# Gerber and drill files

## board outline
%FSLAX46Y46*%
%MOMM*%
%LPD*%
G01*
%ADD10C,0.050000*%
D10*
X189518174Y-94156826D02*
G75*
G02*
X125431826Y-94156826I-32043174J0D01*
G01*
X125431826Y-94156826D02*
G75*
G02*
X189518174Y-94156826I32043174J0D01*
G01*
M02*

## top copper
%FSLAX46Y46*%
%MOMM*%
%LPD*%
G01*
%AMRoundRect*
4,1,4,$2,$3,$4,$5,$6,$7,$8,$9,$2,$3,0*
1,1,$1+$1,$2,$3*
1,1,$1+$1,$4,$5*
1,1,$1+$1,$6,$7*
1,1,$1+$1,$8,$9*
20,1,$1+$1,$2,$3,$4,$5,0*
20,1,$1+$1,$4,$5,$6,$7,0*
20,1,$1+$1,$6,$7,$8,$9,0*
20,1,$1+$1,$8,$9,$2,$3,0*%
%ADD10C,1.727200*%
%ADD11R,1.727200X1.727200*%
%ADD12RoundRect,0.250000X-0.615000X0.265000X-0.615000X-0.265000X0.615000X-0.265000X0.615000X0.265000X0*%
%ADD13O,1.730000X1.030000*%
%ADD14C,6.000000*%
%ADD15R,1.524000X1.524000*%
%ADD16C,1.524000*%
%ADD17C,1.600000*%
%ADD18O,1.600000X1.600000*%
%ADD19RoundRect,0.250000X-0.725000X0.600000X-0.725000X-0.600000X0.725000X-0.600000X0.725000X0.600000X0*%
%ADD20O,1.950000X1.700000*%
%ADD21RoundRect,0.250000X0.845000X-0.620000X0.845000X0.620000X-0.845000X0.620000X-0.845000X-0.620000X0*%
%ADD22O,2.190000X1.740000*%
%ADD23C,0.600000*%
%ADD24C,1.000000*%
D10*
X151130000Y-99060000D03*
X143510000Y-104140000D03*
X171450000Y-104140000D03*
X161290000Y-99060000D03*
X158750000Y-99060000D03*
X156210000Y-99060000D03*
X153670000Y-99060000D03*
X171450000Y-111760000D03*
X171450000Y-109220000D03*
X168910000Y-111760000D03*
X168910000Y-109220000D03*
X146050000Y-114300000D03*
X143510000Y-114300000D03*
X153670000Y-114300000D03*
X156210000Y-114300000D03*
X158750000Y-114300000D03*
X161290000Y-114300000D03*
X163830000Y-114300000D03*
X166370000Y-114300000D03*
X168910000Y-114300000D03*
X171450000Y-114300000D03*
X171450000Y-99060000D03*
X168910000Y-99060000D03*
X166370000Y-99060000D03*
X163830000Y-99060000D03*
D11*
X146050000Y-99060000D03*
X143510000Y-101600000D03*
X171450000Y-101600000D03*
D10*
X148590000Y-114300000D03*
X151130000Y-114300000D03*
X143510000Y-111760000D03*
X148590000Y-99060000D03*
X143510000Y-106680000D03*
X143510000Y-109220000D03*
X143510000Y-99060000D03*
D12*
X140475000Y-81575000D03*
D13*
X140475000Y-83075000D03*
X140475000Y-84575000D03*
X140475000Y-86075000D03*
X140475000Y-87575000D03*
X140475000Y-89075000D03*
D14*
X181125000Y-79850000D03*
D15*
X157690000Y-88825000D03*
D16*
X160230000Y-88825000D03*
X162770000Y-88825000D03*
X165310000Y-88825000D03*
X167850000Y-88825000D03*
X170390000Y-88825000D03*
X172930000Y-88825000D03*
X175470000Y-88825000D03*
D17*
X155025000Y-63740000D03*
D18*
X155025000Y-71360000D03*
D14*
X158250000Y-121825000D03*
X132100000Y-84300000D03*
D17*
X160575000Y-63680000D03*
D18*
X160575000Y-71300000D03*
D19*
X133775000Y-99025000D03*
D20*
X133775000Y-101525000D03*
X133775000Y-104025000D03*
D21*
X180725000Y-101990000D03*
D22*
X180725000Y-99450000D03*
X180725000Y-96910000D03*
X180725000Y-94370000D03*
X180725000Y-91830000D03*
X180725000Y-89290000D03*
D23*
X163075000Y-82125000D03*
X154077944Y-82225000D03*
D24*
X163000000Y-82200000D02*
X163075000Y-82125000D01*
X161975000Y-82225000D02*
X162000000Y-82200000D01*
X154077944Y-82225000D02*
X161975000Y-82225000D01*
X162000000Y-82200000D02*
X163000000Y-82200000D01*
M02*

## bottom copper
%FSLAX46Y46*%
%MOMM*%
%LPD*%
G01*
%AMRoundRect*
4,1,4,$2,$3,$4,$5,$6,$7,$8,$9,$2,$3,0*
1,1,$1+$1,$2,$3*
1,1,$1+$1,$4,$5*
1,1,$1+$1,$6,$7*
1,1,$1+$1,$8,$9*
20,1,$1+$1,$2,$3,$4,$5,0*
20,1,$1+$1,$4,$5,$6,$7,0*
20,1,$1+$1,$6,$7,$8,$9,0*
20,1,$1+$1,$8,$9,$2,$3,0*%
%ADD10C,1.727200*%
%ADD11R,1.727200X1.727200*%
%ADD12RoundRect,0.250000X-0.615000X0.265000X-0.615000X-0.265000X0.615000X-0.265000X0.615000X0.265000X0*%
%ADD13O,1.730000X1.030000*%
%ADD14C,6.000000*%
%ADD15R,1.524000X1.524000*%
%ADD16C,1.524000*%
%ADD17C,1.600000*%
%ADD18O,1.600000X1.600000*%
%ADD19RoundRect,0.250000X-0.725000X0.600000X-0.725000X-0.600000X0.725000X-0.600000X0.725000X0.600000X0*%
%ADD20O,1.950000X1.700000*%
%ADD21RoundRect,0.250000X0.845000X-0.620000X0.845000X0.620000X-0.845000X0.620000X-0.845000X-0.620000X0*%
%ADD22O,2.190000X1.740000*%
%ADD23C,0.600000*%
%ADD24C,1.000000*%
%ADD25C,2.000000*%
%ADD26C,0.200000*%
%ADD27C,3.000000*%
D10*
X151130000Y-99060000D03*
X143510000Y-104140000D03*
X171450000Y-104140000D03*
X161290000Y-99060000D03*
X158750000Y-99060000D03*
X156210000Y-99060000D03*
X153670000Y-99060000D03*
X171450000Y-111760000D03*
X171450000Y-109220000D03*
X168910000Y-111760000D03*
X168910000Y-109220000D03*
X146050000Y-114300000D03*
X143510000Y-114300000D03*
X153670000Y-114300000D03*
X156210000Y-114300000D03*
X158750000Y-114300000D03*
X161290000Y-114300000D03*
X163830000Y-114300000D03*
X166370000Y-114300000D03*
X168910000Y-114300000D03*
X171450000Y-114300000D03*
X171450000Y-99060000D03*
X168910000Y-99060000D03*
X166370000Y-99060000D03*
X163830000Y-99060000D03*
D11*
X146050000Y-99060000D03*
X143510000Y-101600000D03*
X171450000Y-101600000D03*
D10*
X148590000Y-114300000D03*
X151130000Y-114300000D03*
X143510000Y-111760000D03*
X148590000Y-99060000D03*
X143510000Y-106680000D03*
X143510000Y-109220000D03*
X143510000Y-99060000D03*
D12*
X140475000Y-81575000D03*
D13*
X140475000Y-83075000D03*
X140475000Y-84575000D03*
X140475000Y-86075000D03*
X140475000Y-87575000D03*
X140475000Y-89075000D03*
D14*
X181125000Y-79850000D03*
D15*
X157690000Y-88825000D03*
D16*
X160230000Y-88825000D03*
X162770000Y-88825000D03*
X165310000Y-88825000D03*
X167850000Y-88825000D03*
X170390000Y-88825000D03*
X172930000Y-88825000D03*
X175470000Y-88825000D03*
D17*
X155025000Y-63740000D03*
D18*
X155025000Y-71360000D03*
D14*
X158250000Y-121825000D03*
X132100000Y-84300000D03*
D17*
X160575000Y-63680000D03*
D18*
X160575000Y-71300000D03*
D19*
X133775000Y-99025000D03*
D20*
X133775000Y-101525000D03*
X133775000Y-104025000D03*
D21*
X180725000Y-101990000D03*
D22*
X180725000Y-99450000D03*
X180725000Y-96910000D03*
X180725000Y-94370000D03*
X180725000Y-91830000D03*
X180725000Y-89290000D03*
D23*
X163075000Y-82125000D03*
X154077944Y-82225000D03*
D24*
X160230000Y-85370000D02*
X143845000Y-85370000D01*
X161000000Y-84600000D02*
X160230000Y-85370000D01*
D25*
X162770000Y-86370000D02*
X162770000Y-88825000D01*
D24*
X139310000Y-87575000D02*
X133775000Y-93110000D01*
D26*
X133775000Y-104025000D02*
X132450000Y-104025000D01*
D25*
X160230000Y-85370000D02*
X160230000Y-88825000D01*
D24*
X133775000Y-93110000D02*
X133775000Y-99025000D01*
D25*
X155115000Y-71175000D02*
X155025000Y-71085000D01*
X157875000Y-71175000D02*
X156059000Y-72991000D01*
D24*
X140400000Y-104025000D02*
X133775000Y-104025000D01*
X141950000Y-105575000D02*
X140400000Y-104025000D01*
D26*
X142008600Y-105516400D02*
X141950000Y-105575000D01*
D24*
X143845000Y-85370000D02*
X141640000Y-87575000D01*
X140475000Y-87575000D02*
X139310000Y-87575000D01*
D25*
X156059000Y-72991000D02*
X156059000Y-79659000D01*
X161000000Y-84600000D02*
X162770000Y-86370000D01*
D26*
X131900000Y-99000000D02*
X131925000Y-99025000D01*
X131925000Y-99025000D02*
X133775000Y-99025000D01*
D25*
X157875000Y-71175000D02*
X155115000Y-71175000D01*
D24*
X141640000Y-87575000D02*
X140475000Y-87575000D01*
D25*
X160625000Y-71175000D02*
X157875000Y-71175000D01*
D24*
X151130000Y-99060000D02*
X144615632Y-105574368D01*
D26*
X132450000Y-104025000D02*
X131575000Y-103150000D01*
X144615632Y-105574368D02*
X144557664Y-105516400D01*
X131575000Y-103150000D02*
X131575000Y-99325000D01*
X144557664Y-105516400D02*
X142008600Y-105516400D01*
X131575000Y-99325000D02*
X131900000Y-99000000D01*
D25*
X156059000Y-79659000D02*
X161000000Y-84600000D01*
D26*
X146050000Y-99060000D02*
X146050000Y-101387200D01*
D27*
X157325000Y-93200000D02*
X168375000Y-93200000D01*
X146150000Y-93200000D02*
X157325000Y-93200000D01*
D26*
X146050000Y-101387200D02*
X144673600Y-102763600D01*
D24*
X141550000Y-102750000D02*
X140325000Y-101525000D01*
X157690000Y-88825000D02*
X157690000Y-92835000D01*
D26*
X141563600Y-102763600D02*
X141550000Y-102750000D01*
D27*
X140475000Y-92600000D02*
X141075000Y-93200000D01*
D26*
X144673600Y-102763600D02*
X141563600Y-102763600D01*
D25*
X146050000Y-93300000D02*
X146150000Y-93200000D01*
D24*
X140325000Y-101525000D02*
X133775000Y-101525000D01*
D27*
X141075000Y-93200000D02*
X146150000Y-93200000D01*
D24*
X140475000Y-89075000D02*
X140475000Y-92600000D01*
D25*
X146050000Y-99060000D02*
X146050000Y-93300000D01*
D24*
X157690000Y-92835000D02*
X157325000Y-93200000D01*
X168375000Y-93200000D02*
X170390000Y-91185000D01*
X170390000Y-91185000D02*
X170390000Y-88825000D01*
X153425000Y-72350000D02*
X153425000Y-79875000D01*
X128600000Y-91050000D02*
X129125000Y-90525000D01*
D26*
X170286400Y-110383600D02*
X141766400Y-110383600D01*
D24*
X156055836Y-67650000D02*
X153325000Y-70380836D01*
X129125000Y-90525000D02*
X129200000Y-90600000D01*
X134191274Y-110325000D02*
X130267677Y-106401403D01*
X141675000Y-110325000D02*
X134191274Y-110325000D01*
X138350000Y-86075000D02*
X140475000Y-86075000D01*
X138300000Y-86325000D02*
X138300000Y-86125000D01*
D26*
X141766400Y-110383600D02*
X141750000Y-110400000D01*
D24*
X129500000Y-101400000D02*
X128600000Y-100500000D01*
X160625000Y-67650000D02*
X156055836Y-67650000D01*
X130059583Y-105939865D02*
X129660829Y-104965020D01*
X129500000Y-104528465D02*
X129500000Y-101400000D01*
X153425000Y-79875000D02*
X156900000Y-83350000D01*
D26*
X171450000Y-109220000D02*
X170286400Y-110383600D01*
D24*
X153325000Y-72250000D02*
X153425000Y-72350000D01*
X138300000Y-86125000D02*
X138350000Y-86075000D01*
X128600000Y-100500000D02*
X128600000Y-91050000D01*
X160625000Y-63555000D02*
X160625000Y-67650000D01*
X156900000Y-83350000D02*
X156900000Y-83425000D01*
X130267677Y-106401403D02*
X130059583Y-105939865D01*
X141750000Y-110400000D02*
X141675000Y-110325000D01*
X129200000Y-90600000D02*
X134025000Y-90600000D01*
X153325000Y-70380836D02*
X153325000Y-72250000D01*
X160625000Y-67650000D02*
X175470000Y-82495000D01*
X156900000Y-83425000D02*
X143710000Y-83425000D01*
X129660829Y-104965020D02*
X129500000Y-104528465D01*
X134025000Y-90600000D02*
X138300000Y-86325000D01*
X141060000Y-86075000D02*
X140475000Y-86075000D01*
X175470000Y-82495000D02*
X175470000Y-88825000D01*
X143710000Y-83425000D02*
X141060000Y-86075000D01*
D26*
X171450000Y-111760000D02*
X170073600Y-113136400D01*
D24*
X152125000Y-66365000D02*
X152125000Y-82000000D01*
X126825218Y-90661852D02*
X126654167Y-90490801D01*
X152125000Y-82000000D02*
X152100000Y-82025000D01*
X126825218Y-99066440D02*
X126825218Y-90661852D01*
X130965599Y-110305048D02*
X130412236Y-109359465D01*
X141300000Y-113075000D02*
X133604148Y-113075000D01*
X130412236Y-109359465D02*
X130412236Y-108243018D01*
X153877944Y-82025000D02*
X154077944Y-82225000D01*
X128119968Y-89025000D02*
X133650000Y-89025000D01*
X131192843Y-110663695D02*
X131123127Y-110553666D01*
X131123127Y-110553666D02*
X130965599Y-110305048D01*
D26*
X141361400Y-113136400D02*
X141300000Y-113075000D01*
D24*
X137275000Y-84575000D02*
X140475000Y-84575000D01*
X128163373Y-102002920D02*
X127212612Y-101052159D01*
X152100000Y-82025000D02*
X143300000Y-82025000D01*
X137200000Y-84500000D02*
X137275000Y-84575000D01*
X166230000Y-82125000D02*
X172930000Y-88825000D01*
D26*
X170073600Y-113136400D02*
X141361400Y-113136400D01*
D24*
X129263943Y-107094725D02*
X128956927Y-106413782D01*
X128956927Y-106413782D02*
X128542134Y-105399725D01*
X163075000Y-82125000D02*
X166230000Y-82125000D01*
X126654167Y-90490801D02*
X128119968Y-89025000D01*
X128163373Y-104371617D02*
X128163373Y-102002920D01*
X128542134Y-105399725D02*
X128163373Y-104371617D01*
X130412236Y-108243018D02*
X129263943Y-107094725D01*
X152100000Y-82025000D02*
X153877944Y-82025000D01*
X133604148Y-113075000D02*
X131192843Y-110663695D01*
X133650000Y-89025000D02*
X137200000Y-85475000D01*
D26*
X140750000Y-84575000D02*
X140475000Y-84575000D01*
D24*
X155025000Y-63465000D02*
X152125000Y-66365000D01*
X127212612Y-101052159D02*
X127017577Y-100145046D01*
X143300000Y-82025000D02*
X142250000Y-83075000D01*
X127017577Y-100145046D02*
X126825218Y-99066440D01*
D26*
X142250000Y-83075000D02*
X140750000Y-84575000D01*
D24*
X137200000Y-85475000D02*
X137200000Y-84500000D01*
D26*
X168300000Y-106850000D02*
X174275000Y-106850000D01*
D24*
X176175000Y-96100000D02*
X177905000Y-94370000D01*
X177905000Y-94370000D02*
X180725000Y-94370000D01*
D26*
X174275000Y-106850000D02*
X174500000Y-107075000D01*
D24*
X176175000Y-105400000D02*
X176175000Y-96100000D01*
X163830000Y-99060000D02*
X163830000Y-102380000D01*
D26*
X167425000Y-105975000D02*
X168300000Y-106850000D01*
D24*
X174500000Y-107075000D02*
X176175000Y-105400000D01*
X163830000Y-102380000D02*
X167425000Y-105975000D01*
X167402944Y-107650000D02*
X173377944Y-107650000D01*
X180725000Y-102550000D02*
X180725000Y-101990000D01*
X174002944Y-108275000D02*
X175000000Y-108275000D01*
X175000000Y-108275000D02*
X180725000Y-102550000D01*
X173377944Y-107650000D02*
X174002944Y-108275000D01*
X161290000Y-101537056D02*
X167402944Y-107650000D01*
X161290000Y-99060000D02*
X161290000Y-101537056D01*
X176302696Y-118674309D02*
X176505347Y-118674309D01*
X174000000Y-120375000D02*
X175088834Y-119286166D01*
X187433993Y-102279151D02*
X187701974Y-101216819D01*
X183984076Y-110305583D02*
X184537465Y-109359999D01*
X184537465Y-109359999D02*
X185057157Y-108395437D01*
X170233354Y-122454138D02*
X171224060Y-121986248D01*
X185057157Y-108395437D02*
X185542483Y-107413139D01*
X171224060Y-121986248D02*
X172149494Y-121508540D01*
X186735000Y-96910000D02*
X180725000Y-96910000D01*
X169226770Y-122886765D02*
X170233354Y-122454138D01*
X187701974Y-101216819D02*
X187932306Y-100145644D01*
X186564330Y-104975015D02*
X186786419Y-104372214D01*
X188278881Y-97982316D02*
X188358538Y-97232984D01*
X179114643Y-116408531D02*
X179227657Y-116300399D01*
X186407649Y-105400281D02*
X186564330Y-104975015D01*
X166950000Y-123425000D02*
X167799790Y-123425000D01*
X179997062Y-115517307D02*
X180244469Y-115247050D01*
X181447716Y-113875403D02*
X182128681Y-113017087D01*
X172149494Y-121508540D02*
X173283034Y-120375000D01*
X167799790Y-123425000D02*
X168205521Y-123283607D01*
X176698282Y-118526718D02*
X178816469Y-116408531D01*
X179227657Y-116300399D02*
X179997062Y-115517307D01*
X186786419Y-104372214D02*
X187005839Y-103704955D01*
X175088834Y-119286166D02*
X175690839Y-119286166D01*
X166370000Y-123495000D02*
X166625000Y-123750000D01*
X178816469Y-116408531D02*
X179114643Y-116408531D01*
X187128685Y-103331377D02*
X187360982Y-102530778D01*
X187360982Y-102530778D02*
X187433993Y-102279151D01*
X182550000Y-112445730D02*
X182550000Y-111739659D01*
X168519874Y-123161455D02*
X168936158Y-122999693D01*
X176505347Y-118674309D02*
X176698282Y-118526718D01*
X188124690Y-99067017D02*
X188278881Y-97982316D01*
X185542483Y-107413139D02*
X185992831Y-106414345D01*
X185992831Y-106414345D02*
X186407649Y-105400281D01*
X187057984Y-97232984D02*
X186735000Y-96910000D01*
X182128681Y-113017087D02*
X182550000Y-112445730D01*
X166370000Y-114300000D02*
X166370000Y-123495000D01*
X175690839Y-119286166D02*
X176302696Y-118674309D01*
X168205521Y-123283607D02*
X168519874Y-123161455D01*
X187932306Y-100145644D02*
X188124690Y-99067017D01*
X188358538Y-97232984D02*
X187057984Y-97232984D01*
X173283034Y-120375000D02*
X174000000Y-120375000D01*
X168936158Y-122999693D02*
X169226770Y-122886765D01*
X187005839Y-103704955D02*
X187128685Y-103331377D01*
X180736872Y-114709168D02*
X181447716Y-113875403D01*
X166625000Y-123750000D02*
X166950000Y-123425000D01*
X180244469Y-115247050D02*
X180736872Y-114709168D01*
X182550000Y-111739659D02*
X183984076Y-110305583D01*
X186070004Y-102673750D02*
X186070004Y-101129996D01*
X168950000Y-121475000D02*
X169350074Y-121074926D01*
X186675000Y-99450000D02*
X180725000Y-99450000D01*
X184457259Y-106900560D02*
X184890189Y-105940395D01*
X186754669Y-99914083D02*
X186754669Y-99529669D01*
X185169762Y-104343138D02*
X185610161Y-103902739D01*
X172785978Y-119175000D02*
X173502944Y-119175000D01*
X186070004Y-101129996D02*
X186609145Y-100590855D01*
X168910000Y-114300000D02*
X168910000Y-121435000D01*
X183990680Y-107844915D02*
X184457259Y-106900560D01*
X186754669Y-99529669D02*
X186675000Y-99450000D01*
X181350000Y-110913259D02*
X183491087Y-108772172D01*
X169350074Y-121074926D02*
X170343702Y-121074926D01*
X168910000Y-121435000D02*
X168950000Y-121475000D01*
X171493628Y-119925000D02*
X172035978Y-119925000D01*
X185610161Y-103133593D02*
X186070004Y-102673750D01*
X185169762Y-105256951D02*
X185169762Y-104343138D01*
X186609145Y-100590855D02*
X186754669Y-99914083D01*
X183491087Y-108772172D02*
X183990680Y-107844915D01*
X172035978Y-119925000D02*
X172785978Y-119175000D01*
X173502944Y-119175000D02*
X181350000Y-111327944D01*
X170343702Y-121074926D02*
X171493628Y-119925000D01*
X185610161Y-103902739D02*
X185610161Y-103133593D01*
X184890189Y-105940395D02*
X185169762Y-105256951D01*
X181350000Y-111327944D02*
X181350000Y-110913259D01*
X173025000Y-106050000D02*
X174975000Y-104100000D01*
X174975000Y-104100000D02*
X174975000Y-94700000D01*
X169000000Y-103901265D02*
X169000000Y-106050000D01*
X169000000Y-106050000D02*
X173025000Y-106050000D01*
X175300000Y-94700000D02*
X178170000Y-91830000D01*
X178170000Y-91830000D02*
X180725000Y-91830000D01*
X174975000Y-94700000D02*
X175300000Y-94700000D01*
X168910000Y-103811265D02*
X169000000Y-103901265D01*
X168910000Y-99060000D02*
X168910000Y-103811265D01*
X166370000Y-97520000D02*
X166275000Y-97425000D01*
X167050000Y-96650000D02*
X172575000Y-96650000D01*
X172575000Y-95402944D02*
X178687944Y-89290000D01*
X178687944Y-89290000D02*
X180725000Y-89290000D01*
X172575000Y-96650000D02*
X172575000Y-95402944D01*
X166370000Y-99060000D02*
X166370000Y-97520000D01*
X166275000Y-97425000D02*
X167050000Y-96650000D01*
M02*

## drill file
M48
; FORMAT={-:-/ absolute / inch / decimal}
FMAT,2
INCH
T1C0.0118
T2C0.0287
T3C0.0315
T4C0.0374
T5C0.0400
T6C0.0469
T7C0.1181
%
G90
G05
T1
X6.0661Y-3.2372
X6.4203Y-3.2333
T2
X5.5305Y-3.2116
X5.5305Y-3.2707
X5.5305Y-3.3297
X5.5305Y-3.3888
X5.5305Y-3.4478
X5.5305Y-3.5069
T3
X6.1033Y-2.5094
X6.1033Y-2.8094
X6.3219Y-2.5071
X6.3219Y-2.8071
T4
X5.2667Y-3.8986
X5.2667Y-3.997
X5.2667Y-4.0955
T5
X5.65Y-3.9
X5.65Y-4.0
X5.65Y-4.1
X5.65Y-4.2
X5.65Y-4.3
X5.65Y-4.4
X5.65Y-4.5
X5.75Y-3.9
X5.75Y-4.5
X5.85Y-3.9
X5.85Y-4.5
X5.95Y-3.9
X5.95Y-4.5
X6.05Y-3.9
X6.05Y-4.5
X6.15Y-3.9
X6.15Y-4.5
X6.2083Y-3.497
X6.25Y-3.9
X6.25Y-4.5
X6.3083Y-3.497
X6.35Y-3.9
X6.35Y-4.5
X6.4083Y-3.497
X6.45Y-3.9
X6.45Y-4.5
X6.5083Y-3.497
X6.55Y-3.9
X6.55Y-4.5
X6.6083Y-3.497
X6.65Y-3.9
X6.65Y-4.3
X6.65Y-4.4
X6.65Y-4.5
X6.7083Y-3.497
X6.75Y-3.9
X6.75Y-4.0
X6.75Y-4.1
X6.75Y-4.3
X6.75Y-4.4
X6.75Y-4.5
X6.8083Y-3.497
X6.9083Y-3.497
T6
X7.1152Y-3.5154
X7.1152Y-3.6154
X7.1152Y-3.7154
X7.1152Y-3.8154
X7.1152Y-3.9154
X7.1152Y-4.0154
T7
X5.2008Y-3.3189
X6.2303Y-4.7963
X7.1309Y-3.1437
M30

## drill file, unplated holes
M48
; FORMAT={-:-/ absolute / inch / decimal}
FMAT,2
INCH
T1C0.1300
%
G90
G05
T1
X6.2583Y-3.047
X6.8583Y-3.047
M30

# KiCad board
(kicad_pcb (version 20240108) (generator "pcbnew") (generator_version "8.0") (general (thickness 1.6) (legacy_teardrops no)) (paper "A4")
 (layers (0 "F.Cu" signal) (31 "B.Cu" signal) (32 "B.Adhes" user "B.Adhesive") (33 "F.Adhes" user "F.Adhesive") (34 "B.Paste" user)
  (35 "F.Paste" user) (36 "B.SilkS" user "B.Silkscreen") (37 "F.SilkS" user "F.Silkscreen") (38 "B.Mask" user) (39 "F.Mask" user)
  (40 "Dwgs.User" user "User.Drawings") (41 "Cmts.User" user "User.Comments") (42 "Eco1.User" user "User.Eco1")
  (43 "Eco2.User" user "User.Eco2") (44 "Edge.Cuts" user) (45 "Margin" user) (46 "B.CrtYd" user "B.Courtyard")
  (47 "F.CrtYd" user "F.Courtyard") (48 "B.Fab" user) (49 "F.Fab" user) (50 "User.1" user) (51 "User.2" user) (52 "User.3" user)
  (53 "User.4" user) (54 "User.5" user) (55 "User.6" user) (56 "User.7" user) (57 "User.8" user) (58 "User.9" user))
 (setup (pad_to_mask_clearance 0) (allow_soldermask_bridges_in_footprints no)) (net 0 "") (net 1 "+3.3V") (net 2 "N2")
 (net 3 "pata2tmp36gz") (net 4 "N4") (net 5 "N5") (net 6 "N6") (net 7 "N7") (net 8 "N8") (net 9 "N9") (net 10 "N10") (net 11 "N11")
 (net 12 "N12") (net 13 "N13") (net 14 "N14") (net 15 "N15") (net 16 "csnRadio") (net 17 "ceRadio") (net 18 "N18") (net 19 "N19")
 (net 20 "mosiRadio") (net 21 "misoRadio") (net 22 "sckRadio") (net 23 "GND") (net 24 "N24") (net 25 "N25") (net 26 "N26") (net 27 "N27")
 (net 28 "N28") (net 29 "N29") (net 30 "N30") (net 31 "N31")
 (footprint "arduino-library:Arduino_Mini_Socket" (layer "F.Cu") (at 172.72 115.57 90)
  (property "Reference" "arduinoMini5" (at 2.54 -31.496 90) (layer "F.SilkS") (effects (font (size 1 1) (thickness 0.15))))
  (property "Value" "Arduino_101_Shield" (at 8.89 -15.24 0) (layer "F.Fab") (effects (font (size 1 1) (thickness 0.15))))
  (pad "5V1" thru_hole circle (at 16.51 -21.59 90) (size 1.7272 1.7272) (drill 1.016) (layers "*.Cu" "*.Mask") (remove_unused_layers no)
   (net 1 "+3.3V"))
  (pad "5V2" thru_hole circle (at 11.43 -29.21 90) (size 1.7272 1.7272) (drill 1.016) (layers "*.Cu" "*.Mask") (remove_unused_layers no)
   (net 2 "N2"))
  (pad "5V3" thru_hole circle (at 11.43 -1.27 90) (size 1.7272 1.7272) (drill 1.016) (layers "*.Cu" "*.Mask") (remove_unused_layers no))
  (pad "A0" thru_hole circle (at 16.51 -11.43 90) (size 1.7272 1.7272) (drill 1.016) (layers "*.Cu" "*.Mask") (remove_unused_layers no)
   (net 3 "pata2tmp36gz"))
  (pad "A1" thru_hole circle (at 16.51 -13.97 90) (size 1.7272 1.7272) (drill 1.016) (layers "*.Cu" "*.Mask") (remove_unused_layers no)
   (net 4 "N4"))
  (pad "A2" thru_hole circle (at 16.51 -16.51 90) (size 1.7272 1.7272) (drill 1.016) (layers "*.Cu" "*.Mask") (remove_unused_layers no)
   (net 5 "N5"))
  (pad "A3" thru_hole circle (at 16.51 -19.05 90) (size 1.7272 1.7272) (drill 1.016) (layers "*.Cu" "*.Mask") (remove_unused_layers no)
   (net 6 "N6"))
  (pad "A4" thru_hole circle (at 3.81 -1.27 90) (size 1.7272 1.7272) (drill 1.016) (layers "*.Cu" "*.Mask") (remove_unused_layers no)
   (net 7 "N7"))
  (pad "A5" thru_hole circle (at 6.35 -1.27 90) (size 1.7272 1.7272) (drill 1.016) (layers "*.Cu" "*.Mask") (remove_unused_layers no)
   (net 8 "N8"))
  (pad "A6" thru_hole circle (at 3.81 -3.81 90) (size 1.7272 1.7272) (drill 1.016) (layers "*.Cu" "*.Mask") (remove_unused_layers no))
  (pad "A7" thru_hole circle (at 6.35 -3.81 90) (size 1.7272 1.7272) (drill 1.016) (layers "*.Cu" "*.Mask") (remove_unused_layers no))
  (pad "D0" thru_hole circle (at 1.27 -26.67 90) (size 1.7272 1.7272) (drill 1.016) (layers "*.Cu" "*.Mask") (remove_unused_layers no)
   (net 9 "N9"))
  (pad "D1" thru_hole circle (at 1.27 -29.21 90) (size 1.7272 1.7272) (drill 1.016) (layers "*.Cu" "*.Mask") (remove_unused_layers no)
   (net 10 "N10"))
  (pad "D2" thru_hole circle (at 1.27 -19.05 90) (size 1.7272 1.7272) (drill 1.016) (layers "*.Cu" "*.Mask") (remove_unused_layers no)
   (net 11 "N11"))
  (pad "D3" thru_hole circle (at 1.27 -16.51 90) (size 1.7272 1.7272) (drill 1.016) (layers "*.Cu" "*.Mask") (remove_unused_layers no)
   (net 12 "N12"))
  (pad "D4" thru_hole circle (at 1.27 -13.97 90) (size 1.7272 1.7272) (drill 1.016) (layers "*.Cu" "*.Mask") (remove_unused_layers no)
   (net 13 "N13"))
  (pad "D5" thru_hole circle (at 1.27 -11.43 90) (size 1.7272 1.7272) (drill 1.016) (layers "*.Cu" "*.Mask") (remove_unused_layers no)
   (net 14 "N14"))
  (pad "D6" thru_hole circle (at 1.27 -8.89 90) (size 1.7272 1.7272) (drill 1.016) (layers "*.Cu" "*.Mask") (remove_unused_layers no)
   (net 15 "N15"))
  (pad "D7" thru_hole circle (at 1.27 -6.35 90) (size 1.7272 1.7272) (drill 1.016) (layers "*.Cu" "*.Mask") (remove_unused_layers no)
   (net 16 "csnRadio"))
  (pad "D8" thru_hole circle (at 1.27 -3.81 90) (size 1.7272 1.7272) (drill 1.016) (layers "*.Cu" "*.Mask") (remove_unused_layers no)
   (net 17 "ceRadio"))
  (pad "D9" thru_hole circle (at 1.27 -1.27 90) (size 1.7272 1.7272) (drill 1.016) (layers "*.Cu" "*.Mask") (remove_unused_layers no)
   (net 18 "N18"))
  (pad "D10" thru_hole circle (at 16.51 -1.27 90) (size 1.7272 1.7272) (drill 1.016) (layers "*.Cu" "*.Mask") (remove_unused_layers no)
   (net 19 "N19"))
  (pad "D11" thru_hole circle (at 16.51 -3.81 90) (size 1.7272 1.7272) (drill 1.016) (layers "*.Cu" "*.Mask") (remove_unused_layers no)
   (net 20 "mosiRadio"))
  (pad "D12" thru_hole circle (at 16.51 -6.35 90) (size 1.7272 1.7272) (drill 1.016) (layers "*.Cu" "*.Mask") (remove_unused_layers no)
   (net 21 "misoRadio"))
  (pad "D13" thru_hole circle (at 16.51 -8.89 90) (size 1.7272 1.7272) (drill 1.016) (layers "*.Cu" "*.Mask") (remove_unused_layers no)
   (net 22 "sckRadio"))
  (pad "GND2" thru_hole rect (at 16.51 -26.67 90) (size 1.7272 1.7272) (drill 1.016) (layers "*.Cu" "*.Mask") (remove_unused_layers no)
   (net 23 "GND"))
  (pad "GND3" thru_hole rect (at 13.97 -29.21 90) (size 1.7272 1.7272) (drill 1.016) (layers "*.Cu" "*.Mask") (remove_unused_layers no)
   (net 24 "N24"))
  (pad "GND4" thru_hole rect (at 13.97 -1.27 90) (size 1.7272 1.7272) (drill 1.016) (layers "*.Cu" "*.Mask") (remove_unused_layers no)
   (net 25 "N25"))
  (pad "L0" thru_hole circle (at 1.27 -24.13 90) (size 1.7272 1.7272) (drill 1.016) (layers "*.Cu" "*.Mask") (remove_unused_layers no))
  (pad "L1" thru_hole circle (at 1.27 -21.59 90) (size 1.7272 1.7272) (drill 1.016) (layers "*.Cu" "*.Mask") (remove_unused_layers no))
  (pad "L2" thru_hole circle (at 3.81 -29.21 90) (size 1.7272 1.7272) (drill 1.016) (layers "*.Cu" "*.Mask") (remove_unused_layers no))
  (pad "RST2" thru_hole circle (at 16.51 -24.13 90) (size 1.7272 1.7272) (drill 1.016) (layers "*.Cu" "*.Mask") (remove_unused_layers no)
   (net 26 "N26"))
  (pad "RX" thru_hole circle (at 8.89 -29.21 90) (size 1.7272 1.7272) (drill 1.016) (layers "*.Cu" "*.Mask") (remove_unused_layers no))
  (pad "TX" thru_hole circle (at 6.35 -29.21 90) (size 1.7272 1.7272) (drill 1.016) (layers "*.Cu" "*.Mask") (remove_unused_layers no))
  (pad "VIN" thru_hole circle (at 16.51 -29.21 90) (size 1.7272 1.7272) (drill 1.016) (layers "*.Cu" "*.Mask") (remove_unused_layers no)
   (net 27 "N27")))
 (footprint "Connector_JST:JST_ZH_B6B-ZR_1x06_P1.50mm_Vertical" (layer "F.Cu") (at 140.475 81.575 -90)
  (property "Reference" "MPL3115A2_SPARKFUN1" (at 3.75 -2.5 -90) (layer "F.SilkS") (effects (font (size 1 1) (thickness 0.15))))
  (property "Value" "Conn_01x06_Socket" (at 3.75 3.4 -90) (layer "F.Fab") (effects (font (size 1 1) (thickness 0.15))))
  (pad "1" thru_hole roundrect (at 0 0 270) (size 1.03 1.73) (drill 0.73) (layers "*.Cu" "*.Mask") (remove_unused_layers no)
   (roundrect_rratio 0.242718) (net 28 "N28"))
  (pad "2" thru_hole oval (at 1.5 0 270) (size 1.03 1.73) (drill 0.73) (layers "*.Cu" "*.Mask") (remove_unused_layers no) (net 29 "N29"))
  (pad "3" thru_hole oval (at 3 0 270) (size 1.03 1.73) (drill 0.73) (layers "*.Cu" "*.Mask") (remove_unused_layers no) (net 7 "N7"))
  (pad "4" thru_hole oval (at 4.5 0 270) (size 1.03 1.73) (drill 0.73) (layers "*.Cu" "*.Mask") (remove_unused_layers no) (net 8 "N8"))
  (pad "5" thru_hole oval (at 6 0 270) (size 1.03 1.73) (drill 0.73) (layers "*.Cu" "*.Mask") (remove_unused_layers no) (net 1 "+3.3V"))
  (pad "6" thru_hole oval (at 7.5 0 270) (size 1.03 1.73) (drill 0.73) (layers "*.Cu" "*.Mask") (remove_unused_layers no) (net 23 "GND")))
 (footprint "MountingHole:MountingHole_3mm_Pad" (layer "F.Cu") (at 181.125 79.85)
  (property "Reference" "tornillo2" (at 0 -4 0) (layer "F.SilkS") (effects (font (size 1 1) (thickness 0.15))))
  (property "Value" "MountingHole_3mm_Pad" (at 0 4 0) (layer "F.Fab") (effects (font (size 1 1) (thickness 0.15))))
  (pad "2" thru_hole circle (at 0 0) (size 6 6) (drill 3) (layers "*.Cu" "*.Mask") (remove_unused_layers no)))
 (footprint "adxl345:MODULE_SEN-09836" (layer "F.Cu") (at 166.58 82.475)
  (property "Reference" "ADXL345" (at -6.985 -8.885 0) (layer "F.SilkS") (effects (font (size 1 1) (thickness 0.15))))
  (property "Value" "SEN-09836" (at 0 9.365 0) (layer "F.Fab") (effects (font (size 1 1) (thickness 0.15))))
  (pad "" np_thru_hole circle (at -7.62 -5.08) (size 3.302 3.302) (drill 3.302) (layers "*.Cu" "*.Mask"))
  (pad "" np_thru_hole circle (at 7.62 -5.08) (size 3.302 3.302) (drill 3.302) (layers "*.Cu" "*.Mask"))
  (pad "1" thru_hole rect (at -8.89 6.35) (size 1.524 1.524) (drill 1.016) (layers "*.Cu" "*.Mask") (remove_unused_layers no) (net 23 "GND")
   (solder_mask_margin 0.102))
  (pad "2" thru_hole circle (at -6.35 6.35) (size 1.524 1.524) (drill 1.016) (layers "*.Cu" "*.Mask") (remove_unused_layers no)
   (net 1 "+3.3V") (solder_mask_margin 0.102))
  (pad "3" thru_hole circle (at -3.81 6.35) (size 1.524 1.524) (drill 1.016) (layers "*.Cu" "*.Mask") (remove_unused_layers no)
   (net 1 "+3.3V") (solder_mask_margin 0.102))
  (pad "4" thru_hole circle (at -1.27 6.35) (size 1.524 1.524) (drill 1.016) (layers "*.Cu" "*.Mask") (remove_unused_layers no)
   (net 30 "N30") (solder_mask_margin 0.102))
  (pad "5" thru_hole circle (at 1.27 6.35) (size 1.524 1.524) (drill 1.016) (layers "*.Cu" "*.Mask") (remove_unused_layers no)
   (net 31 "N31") (solder_mask_margin 0.102))
  (pad "6" thru_hole circle (at 3.81 6.35) (size 1.524 1.524) (drill 1.016) (layers "*.Cu" "*.Mask") (remove_unused_layers no)
   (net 23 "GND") (solder_mask_margin 0.102))
  (pad "7" thru_hole circle (at 6.35 6.35) (size 1.524 1.524) (drill 1.016) (layers "*.Cu" "*.Mask") (remove_unused_layers no) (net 7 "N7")
   (solder_mask_margin 0.102))
  (pad "8" thru_hole circle (at 8.89 6.35) (size 1.524 1.524) (drill 1.016) (layers "*.Cu" "*.Mask") (remove_unused_layers no) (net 8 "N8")
   (solder_mask_margin 0.102)))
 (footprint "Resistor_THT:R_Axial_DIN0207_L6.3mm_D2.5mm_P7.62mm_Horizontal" (layer "F.Cu") (at 155.025 63.74 -90)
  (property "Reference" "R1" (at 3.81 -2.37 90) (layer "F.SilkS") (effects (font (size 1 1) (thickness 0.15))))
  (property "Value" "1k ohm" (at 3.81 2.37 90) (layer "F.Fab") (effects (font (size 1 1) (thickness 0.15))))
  (pad "1" thru_hole circle (at 0 0 270) (size 1.6 1.6) (drill 0.8) (layers "*.Cu" "*.Mask") (remove_unused_layers no) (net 7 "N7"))
  (pad "2" thru_hole oval (at 7.62 0 270) (size 1.6 1.6) (drill 0.8) (layers "*.Cu" "*.Mask") (remove_unused_layers no) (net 1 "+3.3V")))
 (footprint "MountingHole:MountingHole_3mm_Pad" (layer "F.Cu") (at 158.25 121.825)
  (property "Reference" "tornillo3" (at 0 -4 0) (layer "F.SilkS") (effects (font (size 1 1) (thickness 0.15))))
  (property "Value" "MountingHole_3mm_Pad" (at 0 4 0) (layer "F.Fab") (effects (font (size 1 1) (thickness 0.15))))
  (pad "3" thru_hole circle (at 0 0) (size 6 6) (drill 3) (layers "*.Cu" "*.Mask") (remove_unused_layers no)))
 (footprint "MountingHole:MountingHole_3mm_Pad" (layer "F.Cu") (at 132.1 84.3)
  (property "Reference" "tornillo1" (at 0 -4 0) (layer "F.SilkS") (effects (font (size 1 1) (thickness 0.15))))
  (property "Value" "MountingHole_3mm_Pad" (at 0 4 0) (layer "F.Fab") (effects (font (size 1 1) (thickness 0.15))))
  (pad "1" thru_hole circle (at 0 0) (size 6 6) (drill 3) (layers "*.Cu" "*.Mask") (remove_unused_layers no)))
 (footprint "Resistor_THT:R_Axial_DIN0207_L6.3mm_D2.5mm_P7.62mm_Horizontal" (layer "F.Cu") (at 160.575 63.68 -90)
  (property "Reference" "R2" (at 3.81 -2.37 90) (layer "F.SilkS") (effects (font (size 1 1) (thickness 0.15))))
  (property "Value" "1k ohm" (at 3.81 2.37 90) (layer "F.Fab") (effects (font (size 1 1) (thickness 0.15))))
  (pad "1" thru_hole circle (at 0 0 270) (size 1.6 1.6) (drill 0.8) (layers "*.Cu" "*.Mask") (remove_unused_layers no) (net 8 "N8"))
  (pad "2" thru_hole oval (at 7.62 0 270) (size 1.6 1.6) (drill 0.8) (layers "*.Cu" "*.Mask") (remove_unused_layers no) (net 1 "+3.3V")))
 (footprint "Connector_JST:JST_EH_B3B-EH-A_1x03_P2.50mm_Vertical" (layer "F.Cu") (at 133.775 99.025 -90)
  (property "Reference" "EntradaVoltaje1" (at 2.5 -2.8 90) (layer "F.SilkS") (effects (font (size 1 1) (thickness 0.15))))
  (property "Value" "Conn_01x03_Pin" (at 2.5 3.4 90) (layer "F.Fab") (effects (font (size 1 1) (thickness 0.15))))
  (pad "1" thru_hole roundrect (at 0 0 270) (size 1.7 1.95) (drill 0.95) (layers "*.Cu" "*.Mask") (remove_unused_layers no)
   (roundrect_rratio 0.147059) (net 1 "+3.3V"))
  (pad "2" thru_hole oval (at 2.5 0 270) (size 1.7 1.95) (drill 0.95) (layers "*.Cu" "*.Mask") (remove_unused_layers no) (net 23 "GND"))
  (pad "3" thru_hole oval (at 5 0 270) (size 1.7 1.95) (drill 0.95) (layers "*.Cu" "*.Mask") (remove_unused_layers no) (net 1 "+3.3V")))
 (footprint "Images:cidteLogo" (layer "F.Cu") (at 157.25 95.3 180)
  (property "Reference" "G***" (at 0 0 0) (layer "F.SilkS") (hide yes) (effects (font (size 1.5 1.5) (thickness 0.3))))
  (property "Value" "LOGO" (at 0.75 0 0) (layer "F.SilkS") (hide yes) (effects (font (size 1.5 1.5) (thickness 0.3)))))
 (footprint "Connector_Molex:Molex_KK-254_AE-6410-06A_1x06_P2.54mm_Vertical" (layer "F.Cu") (at 180.725 101.99 90)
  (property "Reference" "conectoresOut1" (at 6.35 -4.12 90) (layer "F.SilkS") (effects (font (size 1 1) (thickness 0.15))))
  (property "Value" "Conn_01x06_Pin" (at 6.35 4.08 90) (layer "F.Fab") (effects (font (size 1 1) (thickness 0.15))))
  (pad "1" thru_hole roundrect (at 0 0 90) (size 1.74 2.19) (drill 1.19) (layers "*.Cu" "*.Mask") (remove_unused_layers no)
   (roundrect_rratio 0.143678) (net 3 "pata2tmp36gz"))
  (pad "2" thru_hole oval (at 2.54 0 90) (size 1.74 2.19) (drill 1.19) (layers "*.Cu" "*.Mask") (remove_unused_layers no) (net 17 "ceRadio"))
  (pad "3" thru_hole oval (at 5.08 0 90) (size 1.74 2.19) (drill 1.19) (layers "*.Cu" "*.Mask") (remove_unused_layers no)
   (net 16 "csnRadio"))
  (pad "4" thru_hole oval (at 7.62 0 90) (size 1.74 2.19) (drill 1.19) (layers "*.Cu" "*.Mask") (remove_unused_layers no)
   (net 22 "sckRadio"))
  (pad "5" thru_hole oval (at 10.16 0 90) (size 1.74 2.19) (drill 1.19) (layers "*.Cu" "*.Mask") (remove_unused_layers no)
   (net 20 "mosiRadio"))
  (pad "6" thru_hole oval (at 12.7 0 90) (size 1.74 2.19) (drill 1.19) (layers "*.Cu" "*.Mask") (remove_unused_layers no)
   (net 21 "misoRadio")))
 (gr_circle (center 157.475 94.156826) (end 179.525 117.406826) (stroke (width 0.05) (type default)) (fill none) (layer "Edge.Cuts"))
 (segment (start 160.23 85.37) (end 143.845 85.37) (width 1) (layer "B.Cu") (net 1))
 (segment (start 161 84.6) (end 160.23 85.37) (width 1) (layer "B.Cu") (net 1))
 (segment (start 162.77 86.37) (end 162.77 88.825) (width 2) (layer "B.Cu") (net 1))
 (segment (start 139.31 87.575) (end 133.775 93.11) (width 1) (layer "B.Cu") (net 1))
 (segment (start 133.775 104.025) (end 132.45 104.025) (width 0.2) (layer "B.Cu") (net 1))
 (segment (start 160.23 85.37) (end 160.23 88.825) (width 2) (layer "B.Cu") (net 1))
 (segment (start 133.775 93.11) (end 133.775 99.025) (width 1) (layer "B.Cu") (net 1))
 (segment (start 155.115 71.175) (end 155.025 71.085) (width 2) (layer "B.Cu") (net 1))
 (segment (start 157.875 71.175) (end 156.059 72.991) (width 2) (layer "B.Cu") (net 1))
 (segment (start 140.4 104.025) (end 133.775 104.025) (width 1) (layer "B.Cu") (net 1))
 (segment (start 141.95 105.575) (end 140.4 104.025) (width 1) (layer "B.Cu") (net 1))
 (segment (start 142.0086 105.5164) (end 141.95 105.575) (width 0.2) (layer "B.Cu") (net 1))
 (segment (start 143.845 85.37) (end 141.64 87.575) (width 1) (layer "B.Cu") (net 1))
 (segment (start 140.475 87.575) (end 139.31 87.575) (width 1) (layer "B.Cu") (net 1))
 (segment (start 156.059 72.991) (end 156.059 79.659) (width 2) (layer "B.Cu") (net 1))
 (segment (start 161 84.6) (end 162.77 86.37) (width 2) (layer "B.Cu") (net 1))
 (segment (start 131.9 99) (end 131.925 99.025) (width 0.2) (layer "B.Cu") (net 1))
 (segment (start 131.925 99.025) (end 133.775 99.025) (width 0.2) (layer "B.Cu") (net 1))
 (segment (start 157.875 71.175) (end 155.115 71.175) (width 2) (layer "B.Cu") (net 1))
 (segment (start 141.64 87.575) (end 140.475 87.575) (width 1) (layer "B.Cu") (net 1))
 (segment (start 160.625 71.175) (end 157.875 71.175) (width 2) (layer "B.Cu") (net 1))
 (segment (start 151.13 99.06) (end 144.615632 105.574368) (width 1) (layer "B.Cu") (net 1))
 (segment (start 132.45 104.025) (end 131.575 103.15) (width 0.2) (layer "B.Cu") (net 1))
 (segment (start 144.615632 105.574368) (end 144.557664 105.5164) (width 0.2) (layer "B.Cu") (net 1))
 (segment (start 131.575 103.15) (end 131.575 99.325) (width 0.2) (layer "B.Cu") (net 1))
 (segment (start 144.557664 105.5164) (end 142.0086 105.5164) (width 0.2) (layer "B.Cu") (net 1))
 (segment (start 131.575 99.325) (end 131.9 99) (width 0.2) (layer "B.Cu") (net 1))
 (segment (start 156.059 79.659) (end 161 84.6) (width 2) (layer "B.Cu") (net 1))
 (segment (start 146.05 99.06) (end 146.05 101.3872) (width 0.2) (layer "B.Cu") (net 23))
 (segment (start 157.325 93.2) (end 168.375 93.2) (width 3) (layer "B.Cu") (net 23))
 (segment (start 146.15 93.2) (end 157.325 93.2) (width 3) (layer "B.Cu") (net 23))
 (segment (start 146.05 101.3872) (end 144.6736 102.7636) (width 0.2) (layer "B.Cu") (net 23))
 (segment (start 141.55 102.75) (end 140.325 101.525) (width 1) (layer "B.Cu") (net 23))
 (segment (start 157.69 88.825) (end 157.69 92.835) (width 1) (layer "B.Cu") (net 23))
 (segment (start 141.5636 102.7636) (end 141.55 102.75) (width 0.2) (layer "B.Cu") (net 23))
 (segment (start 140.475 92.6) (end 141.075 93.2) (width 3) (layer "B.Cu") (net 23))
 (segment (start 144.6736 102.7636) (end 141.5636 102.7636) (width 0.2) (layer "B.Cu") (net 23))
 (segment (start 146.05 93.3) (end 146.15 93.2) (width 2) (layer "B.Cu") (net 23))
 (segment (start 140.325 101.525) (end 133.775 101.525) (width 1) (layer "B.Cu") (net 23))
 (segment (start 141.075 93.2) (end 146.15 93.2) (width 3) (layer "B.Cu") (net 23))
 (segment (start 140.475 89.075) (end 140.475 92.6) (width 1) (layer "B.Cu") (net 23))
 (segment (start 146.05 99.06) (end 146.05 93.3) (width 2) (layer "B.Cu") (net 23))
 (segment (start 157.69 92.835) (end 157.325 93.2) (width 1) (layer "B.Cu") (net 23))
 (segment (start 168.375 93.2) (end 170.39 91.185) (width 1) (layer "B.Cu") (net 23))
 (segment (start 170.39 91.185) (end 170.39 88.825) (width 1) (layer "B.Cu") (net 23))
 (segment (start 153.425 72.35) (end 153.425 79.875) (width 1) (layer "B.Cu") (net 8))
 (segment (start 128.6 91.05) (end 129.125 90.525) (width 1) (layer "B.Cu") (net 8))
 (segment (start 170.2864 110.3836) (end 141.7664 110.3836) (width 0.2) (layer "B.Cu") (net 8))
 (segment (start 156.055836 67.65) (end 153.325 70.380836) (width 1) (layer "B.Cu") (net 8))
 (segment (start 129.125 90.525) (end 129.2 90.6) (width 1) (layer "B.Cu") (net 8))
 (segment (start 134.191274 110.325) (end 130.267677 106.401403) (width 1) (layer "B.Cu") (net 8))
 (segment (start 141.675 110.325) (end 134.191274 110.325) (width 1) (layer "B.Cu") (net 8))
 (segment (start 138.35 86.075) (end 140.475 86.075) (width 1) (layer "B.Cu") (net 8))
 (segment (start 138.3 86.325) (end 138.3 86.125) (width 1) (layer "B.Cu") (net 8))
 (segment (start 141.7664 110.3836) (end 141.75 110.4) (width 0.2) (layer "B.Cu") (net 8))
 (segment (start 129.5 101.4) (end 128.6 100.5) (width 1) (layer "B.Cu") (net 8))
 (segment (start 160.625 67.65) (end 156.055836 67.65) (width 1) (layer "B.Cu") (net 8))
 (segment (start 130.059583 105.939865) (end 129.660829 104.96502) (width 1) (layer "B.Cu") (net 8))
 (segment (start 129.5 104.528465) (end 129.5 101.4) (width 1) (layer "B.Cu") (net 8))
 (segment (start 153.425 79.875) (end 156.9 83.35) (width 1) (layer "B.Cu") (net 8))
 (segment (start 171.45 109.22) (end 170.2864 110.3836) (width 0.2) (layer "B.Cu") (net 8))
 (segment (start 153.325 72.25) (end 153.425 72.35) (width 1) (layer "B.Cu") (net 8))
 (segment (start 138.3 86.125) (end 138.35 86.075) (width 1) (layer "B.Cu") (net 8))
 (segment (start 128.6 100.5) (end 128.6 91.05) (width 1) (layer "B.Cu") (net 8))
 (segment (start 160.625 63.555) (end 160.625 67.65) (width 1) (layer "B.Cu") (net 8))
 (segment (start 156.9 83.35) (end 156.9 83.425) (width 1) (layer "B.Cu") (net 8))
 (segment (start 130.267677 106.401403) (end 130.059583 105.939865) (width 1) (layer "B.Cu") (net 8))
 (segment (start 141.75 110.4) (end 141.675 110.325) (width 1) (layer "B.Cu") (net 8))
 (segment (start 129.2 90.6) (end 134.025 90.6) (width 1) (layer "B.Cu") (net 8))
 (segment (start 153.325 70.380836) (end 153.325 72.25) (width 1) (layer "B.Cu") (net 8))
 (segment (start 160.625 67.65) (end 175.47 82.495) (width 1) (layer "B.Cu") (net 8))
 (segment (start 156.9 83.425) (end 143.71 83.425) (width 1) (layer "B.Cu") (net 8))
 (segment (start 129.660829 104.96502) (end 129.5 104.528465) (width 1) (layer "B.Cu") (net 8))
 (segment (start 134.025 90.6) (end 138.3 86.325) (width 1) (layer "B.Cu") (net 8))
 (segment (start 141.06 86.075) (end 140.475 86.075) (width 1) (layer "B.Cu") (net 8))
 (segment (start 175.47 82.495) (end 175.47 88.825) (width 1) (layer "B.Cu") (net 8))
 (segment (start 143.71 83.425) (end 141.06 86.075) (width 1) (layer "B.Cu") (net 8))
 (segment (start 163 82.2) (end 163.075 82.125) (width 1) (layer "F.Cu") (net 7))
 (segment (start 161.975 82.225) (end 162 82.2) (width 1) (layer "F.Cu") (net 7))
 (segment (start 154.077944 82.225) (end 161.975 82.225) (width 1) (layer "F.Cu") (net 7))
 (segment (start 162 82.2) (end 163 82.2) (width 1) (layer "F.Cu") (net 7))
 (via (at 163.075 82.125) (size 0.6) (drill 0.3) (layers "F.Cu" "B.Cu") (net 7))
 (via (at 154.077944 82.225) (size 0.6) (drill 0.3) (layers "F.Cu" "B.Cu") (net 7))
 (segment (start 171.45 111.76) (end 170.0736 113.1364) (width 0.2) (layer "B.Cu") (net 7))
 (segment (start 152.125 66.365) (end 152.125 82) (width 1) (layer "B.Cu") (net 7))
 (segment (start 126.825218 90.661852) (end 126.654167 90.490801) (width 1) (layer "B.Cu") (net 7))
 (segment (start 152.125 82) (end 152.1 82.025) (width 1) (layer "B.Cu") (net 7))
 (segment (start 126.825218 99.06644) (end 126.825218 90.661852) (width 1) (layer "B.Cu") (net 7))
 (segment (start 130.965599 110.305048) (end 130.412236 109.359465) (width 1) (layer "B.Cu") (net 7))
 (segment (start 141.3 113.075) (end 133.604148 113.075) (width 1) (layer "B.Cu") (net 7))
 (segment (start 130.412236 109.359465) (end 130.412236 108.243018) (width 1) (layer "B.Cu") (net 7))
 (segment (start 153.877944 82.025) (end 154.077944 82.225) (width 1) (layer "B.Cu") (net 7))
 (segment (start 128.119968 89.025) (end 133.65 89.025) (width 1) (layer "B.Cu") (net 7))
 (segment (start 131.192843 110.663695) (end 131.123127 110.553666) (width 1) (layer "B.Cu") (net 7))
 (segment (start 131.123127 110.553666) (end 130.965599 110.305048) (width 1) (layer "B.Cu") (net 7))
 (segment (start 141.3614 113.1364) (end 141.3 113.075) (width 0.2) (layer "B.Cu") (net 7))
 (segment (start 137.275 84.575) (end 140.475 84.575) (width 1) (layer "B.Cu") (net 7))
 (segment (start 128.163373 102.00292) (end 127.212612 101.052159) (width 1) (layer "B.Cu") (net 7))
 (segment (start 152.1 82.025) (end 143.3 82.025) (width 1) (layer "B.Cu") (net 7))
 (segment (start 137.2 84.5) (end 137.275 84.575) (width 1) (layer "B.Cu") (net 7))
 (segment (start 166.23 82.125) (end 172.93 88.825) (width 1) (layer "B.Cu") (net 7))
 (segment (start 170.0736 113.1364) (end 141.3614 113.1364) (width 0.2) (layer "B.Cu") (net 7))
 (segment (start 129.263943 107.094725) (end 128.956927 106.413782) (width 1) (layer "B.Cu") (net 7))
 (segment (start 128.956927 106.413782) (end 128.542134 105.399725) (width 1) (layer "B.Cu") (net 7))
 (segment (start 163.075 82.125) (end 166.23 82.125) (width 1) (layer "B.Cu") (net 7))
 (segment (start 126.654167 90.490801) (end 128.119968 89.025) (width 1) (layer "B.Cu") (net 7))
 (segment (start 128.163373 104.371617) (end 128.163373 102.00292) (width 1) (layer "B.Cu") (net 7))
 (segment (start 128.542134 105.399725) (end 128.163373 104.371617) (width 1) (layer "B.Cu") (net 7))
 (segment (start 130.412236 108.243018) (end 129.263943 107.094725) (width 1) (layer "B.Cu") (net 7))
 (segment (start 152.1 82.025) (end 153.877944 82.025) (width 1) (layer "B.Cu") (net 7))
 (segment (start 133.604148 113.075) (end 131.192843 110.663695) (width 1) (layer "B.Cu") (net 7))
 (segment (start 133.65 89.025) (end 137.2 85.475) (width 1) (layer "B.Cu") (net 7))
 (segment (start 140.75 84.575) (end 140.475 84.575) (width 0.2) (layer "B.Cu") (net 7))
 (segment (start 155.025 63.465) (end 152.125 66.365) (width 1) (layer "B.Cu") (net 7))
 (segment (start 127.212612 101.052159) (end 127.017577 100.145046) (width 1) (layer "B.Cu") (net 7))
 (segment (start 143.3 82.025) (end 142.25 83.075) (width 1) (layer "B.Cu") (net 7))
 (segment (start 127.017577 100.145046) (end 126.825218 99.06644) (width 1) (layer "B.Cu") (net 7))
 (segment (start 142.25 83.075) (end 140.75 84.575) (width 0.2) (layer "B.Cu") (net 7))
 (segment (start 137.2 85.475) (end 137.2 84.5) (width 1) (layer "B.Cu") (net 7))
 (segment (start 168.3 106.85) (end 174.275 106.85) (width 0.2) (layer "B.Cu") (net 22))
 (segment (start 176.175 96.1) (end 177.905 94.37) (width 1) (layer "B.Cu") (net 22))
 (segment (start 177.905 94.37) (end 180.725 94.37) (width 1) (layer "B.Cu") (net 22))
 (segment (start 174.275 106.85) (end 174.5 107.075) (width 0.2) (layer "B.Cu") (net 22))
 (segment (start 176.175 105.4) (end 176.175 96.1) (width 1) (layer "B.Cu") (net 22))
 (segment (start 163.83 99.06) (end 163.83 102.38) (width 1) (layer "B.Cu") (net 22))
 (segment (start 167.425 105.975) (end 168.3 106.85) (width 0.2) (layer "B.Cu") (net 22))
 (segment (start 174.5 107.075) (end 176.175 105.4) (width 1) (layer "B.Cu") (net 22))
 (segment (start 163.83 102.38) (end 167.425 105.975) (width 1) (layer "B.Cu") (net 22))
 (segment (start 167.402944 107.65) (end 173.377944 107.65) (width 1) (layer "B.Cu") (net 3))
 (segment (start 180.725 102.55) (end 180.725 101.99) (width 1) (layer "B.Cu") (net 3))
 (segment (start 174.002944 108.275) (end 175 108.275) (width 1) (layer "B.Cu") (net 3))
 (segment (start 175 108.275) (end 180.725 102.55) (width 1) (layer "B.Cu") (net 3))
 (segment (start 173.377944 107.65) (end 174.002944 108.275) (width 1) (layer "B.Cu") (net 3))
 (segment (start 161.29 101.537056) (end 167.402944 107.65) (width 1) (layer "B.Cu") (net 3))
 (segment (start 161.29 99.06) (end 161.29 101.537056) (width 1) (layer "B.Cu") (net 3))
 (segment (start 176.302696 118.674309) (end 176.505347 118.674309) (width 1) (layer "B.Cu") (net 16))
 (segment (start 174 120.375) (end 175.088834 119.286166) (width 1) (layer "B.Cu") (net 16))
 (segment (start 187.433993 102.279151) (end 187.701974 101.216819) (width 1) (layer "B.Cu") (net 16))
 (segment (start 183.984076 110.305583) (end 184.537465 109.359999) (width 1) (layer "B.Cu") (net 16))
 (segment (start 184.537465 109.359999) (end 185.057157 108.395437) (width 1) (layer "B.Cu") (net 16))
 (segment (start 170.233354 122.454138) (end 171.22406 121.986248) (width 1) (layer "B.Cu") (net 16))
 (segment (start 185.057157 108.395437) (end 185.542483 107.413139) (width 1) (layer "B.Cu") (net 16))
 (segment (start 171.22406 121.986248) (end 172.149494 121.50854) (width 1) (layer "B.Cu") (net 16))
 (segment (start 186.735 96.91) (end 180.725 96.91) (width 1) (layer "B.Cu") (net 16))
 (segment (start 169.22677 122.886765) (end 170.233354 122.454138) (width 1) (layer "B.Cu") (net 16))
 (segment (start 187.701974 101.216819) (end 187.932306 100.145644) (width 1) (layer "B.Cu") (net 16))
 (segment (start 186.56433 104.975015) (end 186.786419 104.372214) (width 1) (layer "B.Cu") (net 16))
 (segment (start 188.278881 97.982316) (end 188.358538 97.232984) (width 1) (layer "B.Cu") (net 16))
 (segment (start 179.114643 116.408531) (end 179.227657 116.300399) (width 1) (layer "B.Cu") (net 16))
 (segment (start 186.407649 105.400281) (end 186.56433 104.975015) (width 1) (layer "B.Cu") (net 16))
 (segment (start 166.95 123.425) (end 167.79979 123.425) (width 1) (layer "B.Cu") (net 16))
 (segment (start 179.997062 115.517307) (end 180.244469 115.24705) (width 1) (layer "B.Cu") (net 16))
 (segment (start 181.447716 113.875403) (end 182.128681 113.017087) (width 1) (layer "B.Cu") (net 16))
 (segment (start 172.149494 121.50854) (end 173.283034 120.375) (width 1) (layer "B.Cu") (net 16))
 (segment (start 167.79979 123.425) (end 168.205521 123.283607) (width 1) (layer "B.Cu") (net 16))
 (segment (start 176.698282 118.526718) (end 178.816469 116.408531) (width 1) (layer "B.Cu") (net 16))
 (segment (start 179.227657 116.300399) (end 179.997062 115.517307) (width 1) (layer "B.Cu") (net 16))
 (segment (start 186.786419 104.372214) (end 187.005839 103.704955) (width 1) (layer "B.Cu") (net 16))
 (segment (start 175.088834 119.286166) (end 175.690839 119.286166) (width 1) (layer "B.Cu") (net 16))
 (segment (start 166.37 123.495) (end 166.625 123.75) (width 1) (layer "B.Cu") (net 16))
 (segment (start 178.816469 116.408531) (end 179.114643 116.408531) (width 1) (layer "B.Cu") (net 16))
 (segment (start 187.128685 103.331377) (end 187.360982 102.530778) (width 1) (layer "B.Cu") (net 16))
 (segment (start 187.360982 102.530778) (end 187.433993 102.279151) (width 1) (layer "B.Cu") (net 16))
 (segment (start 182.55 112.44573) (end 182.55 111.739659) (width 1) (layer "B.Cu") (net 16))
 (segment (start 168.519874 123.161455) (end 168.936158 122.999693) (width 1) (layer "B.Cu") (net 16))
 (segment (start 176.505347 118.674309) (end 176.698282 118.526718) (width 1) (layer "B.Cu") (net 16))
 (segment (start 188.12469 99.067017) (end 188.278881 97.982316) (width 1) (layer "B.Cu") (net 16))
 (segment (start 185.542483 107.413139) (end 185.992831 106.414345) (width 1) (layer "B.Cu") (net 16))
 (segment (start 185.992831 106.414345) (end 186.407649 105.400281) (width 1) (layer "B.Cu") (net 16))
 (segment (start 187.057984 97.232984) (end 186.735 96.91) (width 1) (layer "B.Cu") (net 16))
 (segment (start 182.128681 113.017087) (end 182.55 112.44573) (width 1) (layer "B.Cu") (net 16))
 (segment (start 166.37 114.3) (end 166.37 123.495) (width 1) (layer "B.Cu") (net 16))
 (segment (start 175.690839 119.286166) (end 176.302696 118.674309) (width 1) (layer "B.Cu") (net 16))
 (segment (start 168.205521 123.283607) (end 168.519874 123.161455) (width 1) (layer "B.Cu") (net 16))
 (segment (start 187.932306 100.145644) (end 188.12469 99.067017) (width 1) (layer "B.Cu") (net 16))
 (segment (start 188.358538 97.232984) (end 187.057984 97.232984) (width 1) (layer "B.Cu") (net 16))
 (segment (start 173.283034 120.375) (end 174 120.375) (width 1) (layer "B.Cu") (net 16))
 (segment (start 168.936158 122.999693) (end 169.22677 122.886765) (width 1) (layer "B.Cu") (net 16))
 (segment (start 187.005839 103.704955) (end 187.128685 103.331377) (width 1) (layer "B.Cu") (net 16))
 (segment (start 180.736872 114.709168) (end 181.447716 113.875403) (width 1) (layer "B.Cu") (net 16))
 (segment (start 166.625 123.75) (end 166.95 123.425) (width 1) (layer "B.Cu") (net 16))
 (segment (start 180.244469 115.24705) (end 180.736872 114.709168) (width 1) (layer "B.Cu") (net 16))
 (segment (start 182.55 111.739659) (end 183.984076 110.305583) (width 1) (layer "B.Cu") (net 16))
 (segment (start 186.070004 102.67375) (end 186.070004 101.129996) (width 1) (layer "B.Cu") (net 17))
 (segment (start 168.95 121.475) (end 169.350074 121.074926) (width 1) (layer "B.Cu") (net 17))
 (segment (start 186.675 99.45) (end 180.725 99.45) (width 1) (layer "B.Cu") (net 17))
 (segment (start 184.457259 106.90056) (end 184.890189 105.940395) (width 1) (layer "B.Cu") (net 17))
 (segment (start 186.754669 99.914083) (end 186.754669 99.529669) (width 1) (layer "B.Cu") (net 17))
 (segment (start 185.169762 104.343138) (end 185.610161 103.902739) (width 1) (layer "B.Cu") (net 17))
 (segment (start 172.785978 119.175) (end 173.502944 119.175) (width 1) (layer "B.Cu") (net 17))
 (segment (start 186.070004 101.129996) (end 186.609145 100.590855) (width 1) (layer "B.Cu") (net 17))
 (segment (start 168.91 114.3) (end 168.91 121.435) (width 1) (layer "B.Cu") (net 17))
 (segment (start 183.99068 107.844915) (end 184.457259 106.90056) (width 1) (layer "B.Cu") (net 17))
 (segment (start 186.754669 99.529669) (end 186.675 99.45) (width 1) (layer "B.Cu") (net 17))
 (segment (start 181.35 110.913259) (end 183.491087 108.772172) (width 1) (layer "B.Cu") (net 17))
 (segment (start 169.350074 121.074926) (end 170.343702 121.074926) (width 1) (layer "B.Cu") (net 17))
 (segment (start 168.91 121.435) (end 168.95 121.475) (width 1) (layer "B.Cu") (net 17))
 (segment (start 171.493628 119.925) (end 172.035978 119.925) (width 1) (layer "B.Cu") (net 17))
 (segment (start 185.610161 103.133593) (end 186.070004 102.67375) (width 1) (layer "B.Cu") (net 17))
 (segment (start 185.169762 105.256951) (end 185.169762 104.343138) (width 1) (layer "B.Cu") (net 17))
 (segment (start 186.609145 100.590855) (end 186.754669 99.914083) (width 1) (layer "B.Cu") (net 17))
 (segment (start 183.491087 108.772172) (end 183.99068 107.844915) (width 1) (layer "B.Cu") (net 17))
 (segment (start 172.035978 119.925) (end 172.785978 119.175) (width 1) (layer "B.Cu") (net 17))
 (segment (start 173.502944 119.175) (end 181.35 111.327944) (width 1) (layer "B.Cu") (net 17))
 (segment (start 170.343702 121.074926) (end 171.493628 119.925) (width 1) (layer "B.Cu") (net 17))
 (segment (start 185.610161 103.902739) (end 185.610161 103.133593) (width 1) (layer "B.Cu") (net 17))
 (segment (start 184.890189 105.940395) (end 185.169762 105.256951) (width 1) (layer "B.Cu") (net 17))
 (segment (start 181.35 111.327944) (end 181.35 110.913259) (width 1) (layer "B.Cu") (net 17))
 (segment (start 173.025 106.05) (end 174.975 104.1) (width 1) (layer "B.Cu") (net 20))
 (segment (start 174.975 104.1) (end 174.975 94.7) (width 1) (layer "B.Cu") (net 20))
 (segment (start 169 103.901265) (end 169 106.05) (width 1) (layer "B.Cu") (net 20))
 (segment (start 169 106.05) (end 173.025 106.05) (width 1) (layer "B.Cu") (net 20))
 (segment (start 175.3 94.7) (end 178.17 91.83) (width 1) (layer "B.Cu") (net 20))
 (segment (start 178.17 91.83) (end 180.725 91.83) (width 1) (layer "B.Cu") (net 20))
 (segment (start 174.975 94.7) (end 175.3 94.7) (width 1) (layer "B.Cu") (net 20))
 (segment (start 168.91 103.811265) (end 169 103.901265) (width 1) (layer "B.Cu") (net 20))
 (segment (start 168.91 99.06) (end 168.91 103.811265) (width 1) (layer "B.Cu") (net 20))
 (segment (start 166.37 97.52) (end 166.275 97.425) (width 1) (layer "B.Cu") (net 21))
 (segment (start 167.05 96.65) (end 172.575 96.65) (width 1) (layer "B.Cu") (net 21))
 (segment (start 172.575 95.402944) (end 178.687944 89.29) (width 1) (layer "B.Cu") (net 21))
 (segment (start 178.687944 89.29) (end 180.725 89.29) (width 1) (layer "B.Cu") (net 21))
 (segment (start 172.575 96.65) (end 172.575 95.402944) (width 1) (layer "B.Cu") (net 21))
 (segment (start 166.37 99.06) (end 166.37 97.52) (width 1) (layer "B.Cu") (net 21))
 (segment (start 166.275 97.425) (end 167.05 96.65) (width 1) (layer "B.Cu") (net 21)))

